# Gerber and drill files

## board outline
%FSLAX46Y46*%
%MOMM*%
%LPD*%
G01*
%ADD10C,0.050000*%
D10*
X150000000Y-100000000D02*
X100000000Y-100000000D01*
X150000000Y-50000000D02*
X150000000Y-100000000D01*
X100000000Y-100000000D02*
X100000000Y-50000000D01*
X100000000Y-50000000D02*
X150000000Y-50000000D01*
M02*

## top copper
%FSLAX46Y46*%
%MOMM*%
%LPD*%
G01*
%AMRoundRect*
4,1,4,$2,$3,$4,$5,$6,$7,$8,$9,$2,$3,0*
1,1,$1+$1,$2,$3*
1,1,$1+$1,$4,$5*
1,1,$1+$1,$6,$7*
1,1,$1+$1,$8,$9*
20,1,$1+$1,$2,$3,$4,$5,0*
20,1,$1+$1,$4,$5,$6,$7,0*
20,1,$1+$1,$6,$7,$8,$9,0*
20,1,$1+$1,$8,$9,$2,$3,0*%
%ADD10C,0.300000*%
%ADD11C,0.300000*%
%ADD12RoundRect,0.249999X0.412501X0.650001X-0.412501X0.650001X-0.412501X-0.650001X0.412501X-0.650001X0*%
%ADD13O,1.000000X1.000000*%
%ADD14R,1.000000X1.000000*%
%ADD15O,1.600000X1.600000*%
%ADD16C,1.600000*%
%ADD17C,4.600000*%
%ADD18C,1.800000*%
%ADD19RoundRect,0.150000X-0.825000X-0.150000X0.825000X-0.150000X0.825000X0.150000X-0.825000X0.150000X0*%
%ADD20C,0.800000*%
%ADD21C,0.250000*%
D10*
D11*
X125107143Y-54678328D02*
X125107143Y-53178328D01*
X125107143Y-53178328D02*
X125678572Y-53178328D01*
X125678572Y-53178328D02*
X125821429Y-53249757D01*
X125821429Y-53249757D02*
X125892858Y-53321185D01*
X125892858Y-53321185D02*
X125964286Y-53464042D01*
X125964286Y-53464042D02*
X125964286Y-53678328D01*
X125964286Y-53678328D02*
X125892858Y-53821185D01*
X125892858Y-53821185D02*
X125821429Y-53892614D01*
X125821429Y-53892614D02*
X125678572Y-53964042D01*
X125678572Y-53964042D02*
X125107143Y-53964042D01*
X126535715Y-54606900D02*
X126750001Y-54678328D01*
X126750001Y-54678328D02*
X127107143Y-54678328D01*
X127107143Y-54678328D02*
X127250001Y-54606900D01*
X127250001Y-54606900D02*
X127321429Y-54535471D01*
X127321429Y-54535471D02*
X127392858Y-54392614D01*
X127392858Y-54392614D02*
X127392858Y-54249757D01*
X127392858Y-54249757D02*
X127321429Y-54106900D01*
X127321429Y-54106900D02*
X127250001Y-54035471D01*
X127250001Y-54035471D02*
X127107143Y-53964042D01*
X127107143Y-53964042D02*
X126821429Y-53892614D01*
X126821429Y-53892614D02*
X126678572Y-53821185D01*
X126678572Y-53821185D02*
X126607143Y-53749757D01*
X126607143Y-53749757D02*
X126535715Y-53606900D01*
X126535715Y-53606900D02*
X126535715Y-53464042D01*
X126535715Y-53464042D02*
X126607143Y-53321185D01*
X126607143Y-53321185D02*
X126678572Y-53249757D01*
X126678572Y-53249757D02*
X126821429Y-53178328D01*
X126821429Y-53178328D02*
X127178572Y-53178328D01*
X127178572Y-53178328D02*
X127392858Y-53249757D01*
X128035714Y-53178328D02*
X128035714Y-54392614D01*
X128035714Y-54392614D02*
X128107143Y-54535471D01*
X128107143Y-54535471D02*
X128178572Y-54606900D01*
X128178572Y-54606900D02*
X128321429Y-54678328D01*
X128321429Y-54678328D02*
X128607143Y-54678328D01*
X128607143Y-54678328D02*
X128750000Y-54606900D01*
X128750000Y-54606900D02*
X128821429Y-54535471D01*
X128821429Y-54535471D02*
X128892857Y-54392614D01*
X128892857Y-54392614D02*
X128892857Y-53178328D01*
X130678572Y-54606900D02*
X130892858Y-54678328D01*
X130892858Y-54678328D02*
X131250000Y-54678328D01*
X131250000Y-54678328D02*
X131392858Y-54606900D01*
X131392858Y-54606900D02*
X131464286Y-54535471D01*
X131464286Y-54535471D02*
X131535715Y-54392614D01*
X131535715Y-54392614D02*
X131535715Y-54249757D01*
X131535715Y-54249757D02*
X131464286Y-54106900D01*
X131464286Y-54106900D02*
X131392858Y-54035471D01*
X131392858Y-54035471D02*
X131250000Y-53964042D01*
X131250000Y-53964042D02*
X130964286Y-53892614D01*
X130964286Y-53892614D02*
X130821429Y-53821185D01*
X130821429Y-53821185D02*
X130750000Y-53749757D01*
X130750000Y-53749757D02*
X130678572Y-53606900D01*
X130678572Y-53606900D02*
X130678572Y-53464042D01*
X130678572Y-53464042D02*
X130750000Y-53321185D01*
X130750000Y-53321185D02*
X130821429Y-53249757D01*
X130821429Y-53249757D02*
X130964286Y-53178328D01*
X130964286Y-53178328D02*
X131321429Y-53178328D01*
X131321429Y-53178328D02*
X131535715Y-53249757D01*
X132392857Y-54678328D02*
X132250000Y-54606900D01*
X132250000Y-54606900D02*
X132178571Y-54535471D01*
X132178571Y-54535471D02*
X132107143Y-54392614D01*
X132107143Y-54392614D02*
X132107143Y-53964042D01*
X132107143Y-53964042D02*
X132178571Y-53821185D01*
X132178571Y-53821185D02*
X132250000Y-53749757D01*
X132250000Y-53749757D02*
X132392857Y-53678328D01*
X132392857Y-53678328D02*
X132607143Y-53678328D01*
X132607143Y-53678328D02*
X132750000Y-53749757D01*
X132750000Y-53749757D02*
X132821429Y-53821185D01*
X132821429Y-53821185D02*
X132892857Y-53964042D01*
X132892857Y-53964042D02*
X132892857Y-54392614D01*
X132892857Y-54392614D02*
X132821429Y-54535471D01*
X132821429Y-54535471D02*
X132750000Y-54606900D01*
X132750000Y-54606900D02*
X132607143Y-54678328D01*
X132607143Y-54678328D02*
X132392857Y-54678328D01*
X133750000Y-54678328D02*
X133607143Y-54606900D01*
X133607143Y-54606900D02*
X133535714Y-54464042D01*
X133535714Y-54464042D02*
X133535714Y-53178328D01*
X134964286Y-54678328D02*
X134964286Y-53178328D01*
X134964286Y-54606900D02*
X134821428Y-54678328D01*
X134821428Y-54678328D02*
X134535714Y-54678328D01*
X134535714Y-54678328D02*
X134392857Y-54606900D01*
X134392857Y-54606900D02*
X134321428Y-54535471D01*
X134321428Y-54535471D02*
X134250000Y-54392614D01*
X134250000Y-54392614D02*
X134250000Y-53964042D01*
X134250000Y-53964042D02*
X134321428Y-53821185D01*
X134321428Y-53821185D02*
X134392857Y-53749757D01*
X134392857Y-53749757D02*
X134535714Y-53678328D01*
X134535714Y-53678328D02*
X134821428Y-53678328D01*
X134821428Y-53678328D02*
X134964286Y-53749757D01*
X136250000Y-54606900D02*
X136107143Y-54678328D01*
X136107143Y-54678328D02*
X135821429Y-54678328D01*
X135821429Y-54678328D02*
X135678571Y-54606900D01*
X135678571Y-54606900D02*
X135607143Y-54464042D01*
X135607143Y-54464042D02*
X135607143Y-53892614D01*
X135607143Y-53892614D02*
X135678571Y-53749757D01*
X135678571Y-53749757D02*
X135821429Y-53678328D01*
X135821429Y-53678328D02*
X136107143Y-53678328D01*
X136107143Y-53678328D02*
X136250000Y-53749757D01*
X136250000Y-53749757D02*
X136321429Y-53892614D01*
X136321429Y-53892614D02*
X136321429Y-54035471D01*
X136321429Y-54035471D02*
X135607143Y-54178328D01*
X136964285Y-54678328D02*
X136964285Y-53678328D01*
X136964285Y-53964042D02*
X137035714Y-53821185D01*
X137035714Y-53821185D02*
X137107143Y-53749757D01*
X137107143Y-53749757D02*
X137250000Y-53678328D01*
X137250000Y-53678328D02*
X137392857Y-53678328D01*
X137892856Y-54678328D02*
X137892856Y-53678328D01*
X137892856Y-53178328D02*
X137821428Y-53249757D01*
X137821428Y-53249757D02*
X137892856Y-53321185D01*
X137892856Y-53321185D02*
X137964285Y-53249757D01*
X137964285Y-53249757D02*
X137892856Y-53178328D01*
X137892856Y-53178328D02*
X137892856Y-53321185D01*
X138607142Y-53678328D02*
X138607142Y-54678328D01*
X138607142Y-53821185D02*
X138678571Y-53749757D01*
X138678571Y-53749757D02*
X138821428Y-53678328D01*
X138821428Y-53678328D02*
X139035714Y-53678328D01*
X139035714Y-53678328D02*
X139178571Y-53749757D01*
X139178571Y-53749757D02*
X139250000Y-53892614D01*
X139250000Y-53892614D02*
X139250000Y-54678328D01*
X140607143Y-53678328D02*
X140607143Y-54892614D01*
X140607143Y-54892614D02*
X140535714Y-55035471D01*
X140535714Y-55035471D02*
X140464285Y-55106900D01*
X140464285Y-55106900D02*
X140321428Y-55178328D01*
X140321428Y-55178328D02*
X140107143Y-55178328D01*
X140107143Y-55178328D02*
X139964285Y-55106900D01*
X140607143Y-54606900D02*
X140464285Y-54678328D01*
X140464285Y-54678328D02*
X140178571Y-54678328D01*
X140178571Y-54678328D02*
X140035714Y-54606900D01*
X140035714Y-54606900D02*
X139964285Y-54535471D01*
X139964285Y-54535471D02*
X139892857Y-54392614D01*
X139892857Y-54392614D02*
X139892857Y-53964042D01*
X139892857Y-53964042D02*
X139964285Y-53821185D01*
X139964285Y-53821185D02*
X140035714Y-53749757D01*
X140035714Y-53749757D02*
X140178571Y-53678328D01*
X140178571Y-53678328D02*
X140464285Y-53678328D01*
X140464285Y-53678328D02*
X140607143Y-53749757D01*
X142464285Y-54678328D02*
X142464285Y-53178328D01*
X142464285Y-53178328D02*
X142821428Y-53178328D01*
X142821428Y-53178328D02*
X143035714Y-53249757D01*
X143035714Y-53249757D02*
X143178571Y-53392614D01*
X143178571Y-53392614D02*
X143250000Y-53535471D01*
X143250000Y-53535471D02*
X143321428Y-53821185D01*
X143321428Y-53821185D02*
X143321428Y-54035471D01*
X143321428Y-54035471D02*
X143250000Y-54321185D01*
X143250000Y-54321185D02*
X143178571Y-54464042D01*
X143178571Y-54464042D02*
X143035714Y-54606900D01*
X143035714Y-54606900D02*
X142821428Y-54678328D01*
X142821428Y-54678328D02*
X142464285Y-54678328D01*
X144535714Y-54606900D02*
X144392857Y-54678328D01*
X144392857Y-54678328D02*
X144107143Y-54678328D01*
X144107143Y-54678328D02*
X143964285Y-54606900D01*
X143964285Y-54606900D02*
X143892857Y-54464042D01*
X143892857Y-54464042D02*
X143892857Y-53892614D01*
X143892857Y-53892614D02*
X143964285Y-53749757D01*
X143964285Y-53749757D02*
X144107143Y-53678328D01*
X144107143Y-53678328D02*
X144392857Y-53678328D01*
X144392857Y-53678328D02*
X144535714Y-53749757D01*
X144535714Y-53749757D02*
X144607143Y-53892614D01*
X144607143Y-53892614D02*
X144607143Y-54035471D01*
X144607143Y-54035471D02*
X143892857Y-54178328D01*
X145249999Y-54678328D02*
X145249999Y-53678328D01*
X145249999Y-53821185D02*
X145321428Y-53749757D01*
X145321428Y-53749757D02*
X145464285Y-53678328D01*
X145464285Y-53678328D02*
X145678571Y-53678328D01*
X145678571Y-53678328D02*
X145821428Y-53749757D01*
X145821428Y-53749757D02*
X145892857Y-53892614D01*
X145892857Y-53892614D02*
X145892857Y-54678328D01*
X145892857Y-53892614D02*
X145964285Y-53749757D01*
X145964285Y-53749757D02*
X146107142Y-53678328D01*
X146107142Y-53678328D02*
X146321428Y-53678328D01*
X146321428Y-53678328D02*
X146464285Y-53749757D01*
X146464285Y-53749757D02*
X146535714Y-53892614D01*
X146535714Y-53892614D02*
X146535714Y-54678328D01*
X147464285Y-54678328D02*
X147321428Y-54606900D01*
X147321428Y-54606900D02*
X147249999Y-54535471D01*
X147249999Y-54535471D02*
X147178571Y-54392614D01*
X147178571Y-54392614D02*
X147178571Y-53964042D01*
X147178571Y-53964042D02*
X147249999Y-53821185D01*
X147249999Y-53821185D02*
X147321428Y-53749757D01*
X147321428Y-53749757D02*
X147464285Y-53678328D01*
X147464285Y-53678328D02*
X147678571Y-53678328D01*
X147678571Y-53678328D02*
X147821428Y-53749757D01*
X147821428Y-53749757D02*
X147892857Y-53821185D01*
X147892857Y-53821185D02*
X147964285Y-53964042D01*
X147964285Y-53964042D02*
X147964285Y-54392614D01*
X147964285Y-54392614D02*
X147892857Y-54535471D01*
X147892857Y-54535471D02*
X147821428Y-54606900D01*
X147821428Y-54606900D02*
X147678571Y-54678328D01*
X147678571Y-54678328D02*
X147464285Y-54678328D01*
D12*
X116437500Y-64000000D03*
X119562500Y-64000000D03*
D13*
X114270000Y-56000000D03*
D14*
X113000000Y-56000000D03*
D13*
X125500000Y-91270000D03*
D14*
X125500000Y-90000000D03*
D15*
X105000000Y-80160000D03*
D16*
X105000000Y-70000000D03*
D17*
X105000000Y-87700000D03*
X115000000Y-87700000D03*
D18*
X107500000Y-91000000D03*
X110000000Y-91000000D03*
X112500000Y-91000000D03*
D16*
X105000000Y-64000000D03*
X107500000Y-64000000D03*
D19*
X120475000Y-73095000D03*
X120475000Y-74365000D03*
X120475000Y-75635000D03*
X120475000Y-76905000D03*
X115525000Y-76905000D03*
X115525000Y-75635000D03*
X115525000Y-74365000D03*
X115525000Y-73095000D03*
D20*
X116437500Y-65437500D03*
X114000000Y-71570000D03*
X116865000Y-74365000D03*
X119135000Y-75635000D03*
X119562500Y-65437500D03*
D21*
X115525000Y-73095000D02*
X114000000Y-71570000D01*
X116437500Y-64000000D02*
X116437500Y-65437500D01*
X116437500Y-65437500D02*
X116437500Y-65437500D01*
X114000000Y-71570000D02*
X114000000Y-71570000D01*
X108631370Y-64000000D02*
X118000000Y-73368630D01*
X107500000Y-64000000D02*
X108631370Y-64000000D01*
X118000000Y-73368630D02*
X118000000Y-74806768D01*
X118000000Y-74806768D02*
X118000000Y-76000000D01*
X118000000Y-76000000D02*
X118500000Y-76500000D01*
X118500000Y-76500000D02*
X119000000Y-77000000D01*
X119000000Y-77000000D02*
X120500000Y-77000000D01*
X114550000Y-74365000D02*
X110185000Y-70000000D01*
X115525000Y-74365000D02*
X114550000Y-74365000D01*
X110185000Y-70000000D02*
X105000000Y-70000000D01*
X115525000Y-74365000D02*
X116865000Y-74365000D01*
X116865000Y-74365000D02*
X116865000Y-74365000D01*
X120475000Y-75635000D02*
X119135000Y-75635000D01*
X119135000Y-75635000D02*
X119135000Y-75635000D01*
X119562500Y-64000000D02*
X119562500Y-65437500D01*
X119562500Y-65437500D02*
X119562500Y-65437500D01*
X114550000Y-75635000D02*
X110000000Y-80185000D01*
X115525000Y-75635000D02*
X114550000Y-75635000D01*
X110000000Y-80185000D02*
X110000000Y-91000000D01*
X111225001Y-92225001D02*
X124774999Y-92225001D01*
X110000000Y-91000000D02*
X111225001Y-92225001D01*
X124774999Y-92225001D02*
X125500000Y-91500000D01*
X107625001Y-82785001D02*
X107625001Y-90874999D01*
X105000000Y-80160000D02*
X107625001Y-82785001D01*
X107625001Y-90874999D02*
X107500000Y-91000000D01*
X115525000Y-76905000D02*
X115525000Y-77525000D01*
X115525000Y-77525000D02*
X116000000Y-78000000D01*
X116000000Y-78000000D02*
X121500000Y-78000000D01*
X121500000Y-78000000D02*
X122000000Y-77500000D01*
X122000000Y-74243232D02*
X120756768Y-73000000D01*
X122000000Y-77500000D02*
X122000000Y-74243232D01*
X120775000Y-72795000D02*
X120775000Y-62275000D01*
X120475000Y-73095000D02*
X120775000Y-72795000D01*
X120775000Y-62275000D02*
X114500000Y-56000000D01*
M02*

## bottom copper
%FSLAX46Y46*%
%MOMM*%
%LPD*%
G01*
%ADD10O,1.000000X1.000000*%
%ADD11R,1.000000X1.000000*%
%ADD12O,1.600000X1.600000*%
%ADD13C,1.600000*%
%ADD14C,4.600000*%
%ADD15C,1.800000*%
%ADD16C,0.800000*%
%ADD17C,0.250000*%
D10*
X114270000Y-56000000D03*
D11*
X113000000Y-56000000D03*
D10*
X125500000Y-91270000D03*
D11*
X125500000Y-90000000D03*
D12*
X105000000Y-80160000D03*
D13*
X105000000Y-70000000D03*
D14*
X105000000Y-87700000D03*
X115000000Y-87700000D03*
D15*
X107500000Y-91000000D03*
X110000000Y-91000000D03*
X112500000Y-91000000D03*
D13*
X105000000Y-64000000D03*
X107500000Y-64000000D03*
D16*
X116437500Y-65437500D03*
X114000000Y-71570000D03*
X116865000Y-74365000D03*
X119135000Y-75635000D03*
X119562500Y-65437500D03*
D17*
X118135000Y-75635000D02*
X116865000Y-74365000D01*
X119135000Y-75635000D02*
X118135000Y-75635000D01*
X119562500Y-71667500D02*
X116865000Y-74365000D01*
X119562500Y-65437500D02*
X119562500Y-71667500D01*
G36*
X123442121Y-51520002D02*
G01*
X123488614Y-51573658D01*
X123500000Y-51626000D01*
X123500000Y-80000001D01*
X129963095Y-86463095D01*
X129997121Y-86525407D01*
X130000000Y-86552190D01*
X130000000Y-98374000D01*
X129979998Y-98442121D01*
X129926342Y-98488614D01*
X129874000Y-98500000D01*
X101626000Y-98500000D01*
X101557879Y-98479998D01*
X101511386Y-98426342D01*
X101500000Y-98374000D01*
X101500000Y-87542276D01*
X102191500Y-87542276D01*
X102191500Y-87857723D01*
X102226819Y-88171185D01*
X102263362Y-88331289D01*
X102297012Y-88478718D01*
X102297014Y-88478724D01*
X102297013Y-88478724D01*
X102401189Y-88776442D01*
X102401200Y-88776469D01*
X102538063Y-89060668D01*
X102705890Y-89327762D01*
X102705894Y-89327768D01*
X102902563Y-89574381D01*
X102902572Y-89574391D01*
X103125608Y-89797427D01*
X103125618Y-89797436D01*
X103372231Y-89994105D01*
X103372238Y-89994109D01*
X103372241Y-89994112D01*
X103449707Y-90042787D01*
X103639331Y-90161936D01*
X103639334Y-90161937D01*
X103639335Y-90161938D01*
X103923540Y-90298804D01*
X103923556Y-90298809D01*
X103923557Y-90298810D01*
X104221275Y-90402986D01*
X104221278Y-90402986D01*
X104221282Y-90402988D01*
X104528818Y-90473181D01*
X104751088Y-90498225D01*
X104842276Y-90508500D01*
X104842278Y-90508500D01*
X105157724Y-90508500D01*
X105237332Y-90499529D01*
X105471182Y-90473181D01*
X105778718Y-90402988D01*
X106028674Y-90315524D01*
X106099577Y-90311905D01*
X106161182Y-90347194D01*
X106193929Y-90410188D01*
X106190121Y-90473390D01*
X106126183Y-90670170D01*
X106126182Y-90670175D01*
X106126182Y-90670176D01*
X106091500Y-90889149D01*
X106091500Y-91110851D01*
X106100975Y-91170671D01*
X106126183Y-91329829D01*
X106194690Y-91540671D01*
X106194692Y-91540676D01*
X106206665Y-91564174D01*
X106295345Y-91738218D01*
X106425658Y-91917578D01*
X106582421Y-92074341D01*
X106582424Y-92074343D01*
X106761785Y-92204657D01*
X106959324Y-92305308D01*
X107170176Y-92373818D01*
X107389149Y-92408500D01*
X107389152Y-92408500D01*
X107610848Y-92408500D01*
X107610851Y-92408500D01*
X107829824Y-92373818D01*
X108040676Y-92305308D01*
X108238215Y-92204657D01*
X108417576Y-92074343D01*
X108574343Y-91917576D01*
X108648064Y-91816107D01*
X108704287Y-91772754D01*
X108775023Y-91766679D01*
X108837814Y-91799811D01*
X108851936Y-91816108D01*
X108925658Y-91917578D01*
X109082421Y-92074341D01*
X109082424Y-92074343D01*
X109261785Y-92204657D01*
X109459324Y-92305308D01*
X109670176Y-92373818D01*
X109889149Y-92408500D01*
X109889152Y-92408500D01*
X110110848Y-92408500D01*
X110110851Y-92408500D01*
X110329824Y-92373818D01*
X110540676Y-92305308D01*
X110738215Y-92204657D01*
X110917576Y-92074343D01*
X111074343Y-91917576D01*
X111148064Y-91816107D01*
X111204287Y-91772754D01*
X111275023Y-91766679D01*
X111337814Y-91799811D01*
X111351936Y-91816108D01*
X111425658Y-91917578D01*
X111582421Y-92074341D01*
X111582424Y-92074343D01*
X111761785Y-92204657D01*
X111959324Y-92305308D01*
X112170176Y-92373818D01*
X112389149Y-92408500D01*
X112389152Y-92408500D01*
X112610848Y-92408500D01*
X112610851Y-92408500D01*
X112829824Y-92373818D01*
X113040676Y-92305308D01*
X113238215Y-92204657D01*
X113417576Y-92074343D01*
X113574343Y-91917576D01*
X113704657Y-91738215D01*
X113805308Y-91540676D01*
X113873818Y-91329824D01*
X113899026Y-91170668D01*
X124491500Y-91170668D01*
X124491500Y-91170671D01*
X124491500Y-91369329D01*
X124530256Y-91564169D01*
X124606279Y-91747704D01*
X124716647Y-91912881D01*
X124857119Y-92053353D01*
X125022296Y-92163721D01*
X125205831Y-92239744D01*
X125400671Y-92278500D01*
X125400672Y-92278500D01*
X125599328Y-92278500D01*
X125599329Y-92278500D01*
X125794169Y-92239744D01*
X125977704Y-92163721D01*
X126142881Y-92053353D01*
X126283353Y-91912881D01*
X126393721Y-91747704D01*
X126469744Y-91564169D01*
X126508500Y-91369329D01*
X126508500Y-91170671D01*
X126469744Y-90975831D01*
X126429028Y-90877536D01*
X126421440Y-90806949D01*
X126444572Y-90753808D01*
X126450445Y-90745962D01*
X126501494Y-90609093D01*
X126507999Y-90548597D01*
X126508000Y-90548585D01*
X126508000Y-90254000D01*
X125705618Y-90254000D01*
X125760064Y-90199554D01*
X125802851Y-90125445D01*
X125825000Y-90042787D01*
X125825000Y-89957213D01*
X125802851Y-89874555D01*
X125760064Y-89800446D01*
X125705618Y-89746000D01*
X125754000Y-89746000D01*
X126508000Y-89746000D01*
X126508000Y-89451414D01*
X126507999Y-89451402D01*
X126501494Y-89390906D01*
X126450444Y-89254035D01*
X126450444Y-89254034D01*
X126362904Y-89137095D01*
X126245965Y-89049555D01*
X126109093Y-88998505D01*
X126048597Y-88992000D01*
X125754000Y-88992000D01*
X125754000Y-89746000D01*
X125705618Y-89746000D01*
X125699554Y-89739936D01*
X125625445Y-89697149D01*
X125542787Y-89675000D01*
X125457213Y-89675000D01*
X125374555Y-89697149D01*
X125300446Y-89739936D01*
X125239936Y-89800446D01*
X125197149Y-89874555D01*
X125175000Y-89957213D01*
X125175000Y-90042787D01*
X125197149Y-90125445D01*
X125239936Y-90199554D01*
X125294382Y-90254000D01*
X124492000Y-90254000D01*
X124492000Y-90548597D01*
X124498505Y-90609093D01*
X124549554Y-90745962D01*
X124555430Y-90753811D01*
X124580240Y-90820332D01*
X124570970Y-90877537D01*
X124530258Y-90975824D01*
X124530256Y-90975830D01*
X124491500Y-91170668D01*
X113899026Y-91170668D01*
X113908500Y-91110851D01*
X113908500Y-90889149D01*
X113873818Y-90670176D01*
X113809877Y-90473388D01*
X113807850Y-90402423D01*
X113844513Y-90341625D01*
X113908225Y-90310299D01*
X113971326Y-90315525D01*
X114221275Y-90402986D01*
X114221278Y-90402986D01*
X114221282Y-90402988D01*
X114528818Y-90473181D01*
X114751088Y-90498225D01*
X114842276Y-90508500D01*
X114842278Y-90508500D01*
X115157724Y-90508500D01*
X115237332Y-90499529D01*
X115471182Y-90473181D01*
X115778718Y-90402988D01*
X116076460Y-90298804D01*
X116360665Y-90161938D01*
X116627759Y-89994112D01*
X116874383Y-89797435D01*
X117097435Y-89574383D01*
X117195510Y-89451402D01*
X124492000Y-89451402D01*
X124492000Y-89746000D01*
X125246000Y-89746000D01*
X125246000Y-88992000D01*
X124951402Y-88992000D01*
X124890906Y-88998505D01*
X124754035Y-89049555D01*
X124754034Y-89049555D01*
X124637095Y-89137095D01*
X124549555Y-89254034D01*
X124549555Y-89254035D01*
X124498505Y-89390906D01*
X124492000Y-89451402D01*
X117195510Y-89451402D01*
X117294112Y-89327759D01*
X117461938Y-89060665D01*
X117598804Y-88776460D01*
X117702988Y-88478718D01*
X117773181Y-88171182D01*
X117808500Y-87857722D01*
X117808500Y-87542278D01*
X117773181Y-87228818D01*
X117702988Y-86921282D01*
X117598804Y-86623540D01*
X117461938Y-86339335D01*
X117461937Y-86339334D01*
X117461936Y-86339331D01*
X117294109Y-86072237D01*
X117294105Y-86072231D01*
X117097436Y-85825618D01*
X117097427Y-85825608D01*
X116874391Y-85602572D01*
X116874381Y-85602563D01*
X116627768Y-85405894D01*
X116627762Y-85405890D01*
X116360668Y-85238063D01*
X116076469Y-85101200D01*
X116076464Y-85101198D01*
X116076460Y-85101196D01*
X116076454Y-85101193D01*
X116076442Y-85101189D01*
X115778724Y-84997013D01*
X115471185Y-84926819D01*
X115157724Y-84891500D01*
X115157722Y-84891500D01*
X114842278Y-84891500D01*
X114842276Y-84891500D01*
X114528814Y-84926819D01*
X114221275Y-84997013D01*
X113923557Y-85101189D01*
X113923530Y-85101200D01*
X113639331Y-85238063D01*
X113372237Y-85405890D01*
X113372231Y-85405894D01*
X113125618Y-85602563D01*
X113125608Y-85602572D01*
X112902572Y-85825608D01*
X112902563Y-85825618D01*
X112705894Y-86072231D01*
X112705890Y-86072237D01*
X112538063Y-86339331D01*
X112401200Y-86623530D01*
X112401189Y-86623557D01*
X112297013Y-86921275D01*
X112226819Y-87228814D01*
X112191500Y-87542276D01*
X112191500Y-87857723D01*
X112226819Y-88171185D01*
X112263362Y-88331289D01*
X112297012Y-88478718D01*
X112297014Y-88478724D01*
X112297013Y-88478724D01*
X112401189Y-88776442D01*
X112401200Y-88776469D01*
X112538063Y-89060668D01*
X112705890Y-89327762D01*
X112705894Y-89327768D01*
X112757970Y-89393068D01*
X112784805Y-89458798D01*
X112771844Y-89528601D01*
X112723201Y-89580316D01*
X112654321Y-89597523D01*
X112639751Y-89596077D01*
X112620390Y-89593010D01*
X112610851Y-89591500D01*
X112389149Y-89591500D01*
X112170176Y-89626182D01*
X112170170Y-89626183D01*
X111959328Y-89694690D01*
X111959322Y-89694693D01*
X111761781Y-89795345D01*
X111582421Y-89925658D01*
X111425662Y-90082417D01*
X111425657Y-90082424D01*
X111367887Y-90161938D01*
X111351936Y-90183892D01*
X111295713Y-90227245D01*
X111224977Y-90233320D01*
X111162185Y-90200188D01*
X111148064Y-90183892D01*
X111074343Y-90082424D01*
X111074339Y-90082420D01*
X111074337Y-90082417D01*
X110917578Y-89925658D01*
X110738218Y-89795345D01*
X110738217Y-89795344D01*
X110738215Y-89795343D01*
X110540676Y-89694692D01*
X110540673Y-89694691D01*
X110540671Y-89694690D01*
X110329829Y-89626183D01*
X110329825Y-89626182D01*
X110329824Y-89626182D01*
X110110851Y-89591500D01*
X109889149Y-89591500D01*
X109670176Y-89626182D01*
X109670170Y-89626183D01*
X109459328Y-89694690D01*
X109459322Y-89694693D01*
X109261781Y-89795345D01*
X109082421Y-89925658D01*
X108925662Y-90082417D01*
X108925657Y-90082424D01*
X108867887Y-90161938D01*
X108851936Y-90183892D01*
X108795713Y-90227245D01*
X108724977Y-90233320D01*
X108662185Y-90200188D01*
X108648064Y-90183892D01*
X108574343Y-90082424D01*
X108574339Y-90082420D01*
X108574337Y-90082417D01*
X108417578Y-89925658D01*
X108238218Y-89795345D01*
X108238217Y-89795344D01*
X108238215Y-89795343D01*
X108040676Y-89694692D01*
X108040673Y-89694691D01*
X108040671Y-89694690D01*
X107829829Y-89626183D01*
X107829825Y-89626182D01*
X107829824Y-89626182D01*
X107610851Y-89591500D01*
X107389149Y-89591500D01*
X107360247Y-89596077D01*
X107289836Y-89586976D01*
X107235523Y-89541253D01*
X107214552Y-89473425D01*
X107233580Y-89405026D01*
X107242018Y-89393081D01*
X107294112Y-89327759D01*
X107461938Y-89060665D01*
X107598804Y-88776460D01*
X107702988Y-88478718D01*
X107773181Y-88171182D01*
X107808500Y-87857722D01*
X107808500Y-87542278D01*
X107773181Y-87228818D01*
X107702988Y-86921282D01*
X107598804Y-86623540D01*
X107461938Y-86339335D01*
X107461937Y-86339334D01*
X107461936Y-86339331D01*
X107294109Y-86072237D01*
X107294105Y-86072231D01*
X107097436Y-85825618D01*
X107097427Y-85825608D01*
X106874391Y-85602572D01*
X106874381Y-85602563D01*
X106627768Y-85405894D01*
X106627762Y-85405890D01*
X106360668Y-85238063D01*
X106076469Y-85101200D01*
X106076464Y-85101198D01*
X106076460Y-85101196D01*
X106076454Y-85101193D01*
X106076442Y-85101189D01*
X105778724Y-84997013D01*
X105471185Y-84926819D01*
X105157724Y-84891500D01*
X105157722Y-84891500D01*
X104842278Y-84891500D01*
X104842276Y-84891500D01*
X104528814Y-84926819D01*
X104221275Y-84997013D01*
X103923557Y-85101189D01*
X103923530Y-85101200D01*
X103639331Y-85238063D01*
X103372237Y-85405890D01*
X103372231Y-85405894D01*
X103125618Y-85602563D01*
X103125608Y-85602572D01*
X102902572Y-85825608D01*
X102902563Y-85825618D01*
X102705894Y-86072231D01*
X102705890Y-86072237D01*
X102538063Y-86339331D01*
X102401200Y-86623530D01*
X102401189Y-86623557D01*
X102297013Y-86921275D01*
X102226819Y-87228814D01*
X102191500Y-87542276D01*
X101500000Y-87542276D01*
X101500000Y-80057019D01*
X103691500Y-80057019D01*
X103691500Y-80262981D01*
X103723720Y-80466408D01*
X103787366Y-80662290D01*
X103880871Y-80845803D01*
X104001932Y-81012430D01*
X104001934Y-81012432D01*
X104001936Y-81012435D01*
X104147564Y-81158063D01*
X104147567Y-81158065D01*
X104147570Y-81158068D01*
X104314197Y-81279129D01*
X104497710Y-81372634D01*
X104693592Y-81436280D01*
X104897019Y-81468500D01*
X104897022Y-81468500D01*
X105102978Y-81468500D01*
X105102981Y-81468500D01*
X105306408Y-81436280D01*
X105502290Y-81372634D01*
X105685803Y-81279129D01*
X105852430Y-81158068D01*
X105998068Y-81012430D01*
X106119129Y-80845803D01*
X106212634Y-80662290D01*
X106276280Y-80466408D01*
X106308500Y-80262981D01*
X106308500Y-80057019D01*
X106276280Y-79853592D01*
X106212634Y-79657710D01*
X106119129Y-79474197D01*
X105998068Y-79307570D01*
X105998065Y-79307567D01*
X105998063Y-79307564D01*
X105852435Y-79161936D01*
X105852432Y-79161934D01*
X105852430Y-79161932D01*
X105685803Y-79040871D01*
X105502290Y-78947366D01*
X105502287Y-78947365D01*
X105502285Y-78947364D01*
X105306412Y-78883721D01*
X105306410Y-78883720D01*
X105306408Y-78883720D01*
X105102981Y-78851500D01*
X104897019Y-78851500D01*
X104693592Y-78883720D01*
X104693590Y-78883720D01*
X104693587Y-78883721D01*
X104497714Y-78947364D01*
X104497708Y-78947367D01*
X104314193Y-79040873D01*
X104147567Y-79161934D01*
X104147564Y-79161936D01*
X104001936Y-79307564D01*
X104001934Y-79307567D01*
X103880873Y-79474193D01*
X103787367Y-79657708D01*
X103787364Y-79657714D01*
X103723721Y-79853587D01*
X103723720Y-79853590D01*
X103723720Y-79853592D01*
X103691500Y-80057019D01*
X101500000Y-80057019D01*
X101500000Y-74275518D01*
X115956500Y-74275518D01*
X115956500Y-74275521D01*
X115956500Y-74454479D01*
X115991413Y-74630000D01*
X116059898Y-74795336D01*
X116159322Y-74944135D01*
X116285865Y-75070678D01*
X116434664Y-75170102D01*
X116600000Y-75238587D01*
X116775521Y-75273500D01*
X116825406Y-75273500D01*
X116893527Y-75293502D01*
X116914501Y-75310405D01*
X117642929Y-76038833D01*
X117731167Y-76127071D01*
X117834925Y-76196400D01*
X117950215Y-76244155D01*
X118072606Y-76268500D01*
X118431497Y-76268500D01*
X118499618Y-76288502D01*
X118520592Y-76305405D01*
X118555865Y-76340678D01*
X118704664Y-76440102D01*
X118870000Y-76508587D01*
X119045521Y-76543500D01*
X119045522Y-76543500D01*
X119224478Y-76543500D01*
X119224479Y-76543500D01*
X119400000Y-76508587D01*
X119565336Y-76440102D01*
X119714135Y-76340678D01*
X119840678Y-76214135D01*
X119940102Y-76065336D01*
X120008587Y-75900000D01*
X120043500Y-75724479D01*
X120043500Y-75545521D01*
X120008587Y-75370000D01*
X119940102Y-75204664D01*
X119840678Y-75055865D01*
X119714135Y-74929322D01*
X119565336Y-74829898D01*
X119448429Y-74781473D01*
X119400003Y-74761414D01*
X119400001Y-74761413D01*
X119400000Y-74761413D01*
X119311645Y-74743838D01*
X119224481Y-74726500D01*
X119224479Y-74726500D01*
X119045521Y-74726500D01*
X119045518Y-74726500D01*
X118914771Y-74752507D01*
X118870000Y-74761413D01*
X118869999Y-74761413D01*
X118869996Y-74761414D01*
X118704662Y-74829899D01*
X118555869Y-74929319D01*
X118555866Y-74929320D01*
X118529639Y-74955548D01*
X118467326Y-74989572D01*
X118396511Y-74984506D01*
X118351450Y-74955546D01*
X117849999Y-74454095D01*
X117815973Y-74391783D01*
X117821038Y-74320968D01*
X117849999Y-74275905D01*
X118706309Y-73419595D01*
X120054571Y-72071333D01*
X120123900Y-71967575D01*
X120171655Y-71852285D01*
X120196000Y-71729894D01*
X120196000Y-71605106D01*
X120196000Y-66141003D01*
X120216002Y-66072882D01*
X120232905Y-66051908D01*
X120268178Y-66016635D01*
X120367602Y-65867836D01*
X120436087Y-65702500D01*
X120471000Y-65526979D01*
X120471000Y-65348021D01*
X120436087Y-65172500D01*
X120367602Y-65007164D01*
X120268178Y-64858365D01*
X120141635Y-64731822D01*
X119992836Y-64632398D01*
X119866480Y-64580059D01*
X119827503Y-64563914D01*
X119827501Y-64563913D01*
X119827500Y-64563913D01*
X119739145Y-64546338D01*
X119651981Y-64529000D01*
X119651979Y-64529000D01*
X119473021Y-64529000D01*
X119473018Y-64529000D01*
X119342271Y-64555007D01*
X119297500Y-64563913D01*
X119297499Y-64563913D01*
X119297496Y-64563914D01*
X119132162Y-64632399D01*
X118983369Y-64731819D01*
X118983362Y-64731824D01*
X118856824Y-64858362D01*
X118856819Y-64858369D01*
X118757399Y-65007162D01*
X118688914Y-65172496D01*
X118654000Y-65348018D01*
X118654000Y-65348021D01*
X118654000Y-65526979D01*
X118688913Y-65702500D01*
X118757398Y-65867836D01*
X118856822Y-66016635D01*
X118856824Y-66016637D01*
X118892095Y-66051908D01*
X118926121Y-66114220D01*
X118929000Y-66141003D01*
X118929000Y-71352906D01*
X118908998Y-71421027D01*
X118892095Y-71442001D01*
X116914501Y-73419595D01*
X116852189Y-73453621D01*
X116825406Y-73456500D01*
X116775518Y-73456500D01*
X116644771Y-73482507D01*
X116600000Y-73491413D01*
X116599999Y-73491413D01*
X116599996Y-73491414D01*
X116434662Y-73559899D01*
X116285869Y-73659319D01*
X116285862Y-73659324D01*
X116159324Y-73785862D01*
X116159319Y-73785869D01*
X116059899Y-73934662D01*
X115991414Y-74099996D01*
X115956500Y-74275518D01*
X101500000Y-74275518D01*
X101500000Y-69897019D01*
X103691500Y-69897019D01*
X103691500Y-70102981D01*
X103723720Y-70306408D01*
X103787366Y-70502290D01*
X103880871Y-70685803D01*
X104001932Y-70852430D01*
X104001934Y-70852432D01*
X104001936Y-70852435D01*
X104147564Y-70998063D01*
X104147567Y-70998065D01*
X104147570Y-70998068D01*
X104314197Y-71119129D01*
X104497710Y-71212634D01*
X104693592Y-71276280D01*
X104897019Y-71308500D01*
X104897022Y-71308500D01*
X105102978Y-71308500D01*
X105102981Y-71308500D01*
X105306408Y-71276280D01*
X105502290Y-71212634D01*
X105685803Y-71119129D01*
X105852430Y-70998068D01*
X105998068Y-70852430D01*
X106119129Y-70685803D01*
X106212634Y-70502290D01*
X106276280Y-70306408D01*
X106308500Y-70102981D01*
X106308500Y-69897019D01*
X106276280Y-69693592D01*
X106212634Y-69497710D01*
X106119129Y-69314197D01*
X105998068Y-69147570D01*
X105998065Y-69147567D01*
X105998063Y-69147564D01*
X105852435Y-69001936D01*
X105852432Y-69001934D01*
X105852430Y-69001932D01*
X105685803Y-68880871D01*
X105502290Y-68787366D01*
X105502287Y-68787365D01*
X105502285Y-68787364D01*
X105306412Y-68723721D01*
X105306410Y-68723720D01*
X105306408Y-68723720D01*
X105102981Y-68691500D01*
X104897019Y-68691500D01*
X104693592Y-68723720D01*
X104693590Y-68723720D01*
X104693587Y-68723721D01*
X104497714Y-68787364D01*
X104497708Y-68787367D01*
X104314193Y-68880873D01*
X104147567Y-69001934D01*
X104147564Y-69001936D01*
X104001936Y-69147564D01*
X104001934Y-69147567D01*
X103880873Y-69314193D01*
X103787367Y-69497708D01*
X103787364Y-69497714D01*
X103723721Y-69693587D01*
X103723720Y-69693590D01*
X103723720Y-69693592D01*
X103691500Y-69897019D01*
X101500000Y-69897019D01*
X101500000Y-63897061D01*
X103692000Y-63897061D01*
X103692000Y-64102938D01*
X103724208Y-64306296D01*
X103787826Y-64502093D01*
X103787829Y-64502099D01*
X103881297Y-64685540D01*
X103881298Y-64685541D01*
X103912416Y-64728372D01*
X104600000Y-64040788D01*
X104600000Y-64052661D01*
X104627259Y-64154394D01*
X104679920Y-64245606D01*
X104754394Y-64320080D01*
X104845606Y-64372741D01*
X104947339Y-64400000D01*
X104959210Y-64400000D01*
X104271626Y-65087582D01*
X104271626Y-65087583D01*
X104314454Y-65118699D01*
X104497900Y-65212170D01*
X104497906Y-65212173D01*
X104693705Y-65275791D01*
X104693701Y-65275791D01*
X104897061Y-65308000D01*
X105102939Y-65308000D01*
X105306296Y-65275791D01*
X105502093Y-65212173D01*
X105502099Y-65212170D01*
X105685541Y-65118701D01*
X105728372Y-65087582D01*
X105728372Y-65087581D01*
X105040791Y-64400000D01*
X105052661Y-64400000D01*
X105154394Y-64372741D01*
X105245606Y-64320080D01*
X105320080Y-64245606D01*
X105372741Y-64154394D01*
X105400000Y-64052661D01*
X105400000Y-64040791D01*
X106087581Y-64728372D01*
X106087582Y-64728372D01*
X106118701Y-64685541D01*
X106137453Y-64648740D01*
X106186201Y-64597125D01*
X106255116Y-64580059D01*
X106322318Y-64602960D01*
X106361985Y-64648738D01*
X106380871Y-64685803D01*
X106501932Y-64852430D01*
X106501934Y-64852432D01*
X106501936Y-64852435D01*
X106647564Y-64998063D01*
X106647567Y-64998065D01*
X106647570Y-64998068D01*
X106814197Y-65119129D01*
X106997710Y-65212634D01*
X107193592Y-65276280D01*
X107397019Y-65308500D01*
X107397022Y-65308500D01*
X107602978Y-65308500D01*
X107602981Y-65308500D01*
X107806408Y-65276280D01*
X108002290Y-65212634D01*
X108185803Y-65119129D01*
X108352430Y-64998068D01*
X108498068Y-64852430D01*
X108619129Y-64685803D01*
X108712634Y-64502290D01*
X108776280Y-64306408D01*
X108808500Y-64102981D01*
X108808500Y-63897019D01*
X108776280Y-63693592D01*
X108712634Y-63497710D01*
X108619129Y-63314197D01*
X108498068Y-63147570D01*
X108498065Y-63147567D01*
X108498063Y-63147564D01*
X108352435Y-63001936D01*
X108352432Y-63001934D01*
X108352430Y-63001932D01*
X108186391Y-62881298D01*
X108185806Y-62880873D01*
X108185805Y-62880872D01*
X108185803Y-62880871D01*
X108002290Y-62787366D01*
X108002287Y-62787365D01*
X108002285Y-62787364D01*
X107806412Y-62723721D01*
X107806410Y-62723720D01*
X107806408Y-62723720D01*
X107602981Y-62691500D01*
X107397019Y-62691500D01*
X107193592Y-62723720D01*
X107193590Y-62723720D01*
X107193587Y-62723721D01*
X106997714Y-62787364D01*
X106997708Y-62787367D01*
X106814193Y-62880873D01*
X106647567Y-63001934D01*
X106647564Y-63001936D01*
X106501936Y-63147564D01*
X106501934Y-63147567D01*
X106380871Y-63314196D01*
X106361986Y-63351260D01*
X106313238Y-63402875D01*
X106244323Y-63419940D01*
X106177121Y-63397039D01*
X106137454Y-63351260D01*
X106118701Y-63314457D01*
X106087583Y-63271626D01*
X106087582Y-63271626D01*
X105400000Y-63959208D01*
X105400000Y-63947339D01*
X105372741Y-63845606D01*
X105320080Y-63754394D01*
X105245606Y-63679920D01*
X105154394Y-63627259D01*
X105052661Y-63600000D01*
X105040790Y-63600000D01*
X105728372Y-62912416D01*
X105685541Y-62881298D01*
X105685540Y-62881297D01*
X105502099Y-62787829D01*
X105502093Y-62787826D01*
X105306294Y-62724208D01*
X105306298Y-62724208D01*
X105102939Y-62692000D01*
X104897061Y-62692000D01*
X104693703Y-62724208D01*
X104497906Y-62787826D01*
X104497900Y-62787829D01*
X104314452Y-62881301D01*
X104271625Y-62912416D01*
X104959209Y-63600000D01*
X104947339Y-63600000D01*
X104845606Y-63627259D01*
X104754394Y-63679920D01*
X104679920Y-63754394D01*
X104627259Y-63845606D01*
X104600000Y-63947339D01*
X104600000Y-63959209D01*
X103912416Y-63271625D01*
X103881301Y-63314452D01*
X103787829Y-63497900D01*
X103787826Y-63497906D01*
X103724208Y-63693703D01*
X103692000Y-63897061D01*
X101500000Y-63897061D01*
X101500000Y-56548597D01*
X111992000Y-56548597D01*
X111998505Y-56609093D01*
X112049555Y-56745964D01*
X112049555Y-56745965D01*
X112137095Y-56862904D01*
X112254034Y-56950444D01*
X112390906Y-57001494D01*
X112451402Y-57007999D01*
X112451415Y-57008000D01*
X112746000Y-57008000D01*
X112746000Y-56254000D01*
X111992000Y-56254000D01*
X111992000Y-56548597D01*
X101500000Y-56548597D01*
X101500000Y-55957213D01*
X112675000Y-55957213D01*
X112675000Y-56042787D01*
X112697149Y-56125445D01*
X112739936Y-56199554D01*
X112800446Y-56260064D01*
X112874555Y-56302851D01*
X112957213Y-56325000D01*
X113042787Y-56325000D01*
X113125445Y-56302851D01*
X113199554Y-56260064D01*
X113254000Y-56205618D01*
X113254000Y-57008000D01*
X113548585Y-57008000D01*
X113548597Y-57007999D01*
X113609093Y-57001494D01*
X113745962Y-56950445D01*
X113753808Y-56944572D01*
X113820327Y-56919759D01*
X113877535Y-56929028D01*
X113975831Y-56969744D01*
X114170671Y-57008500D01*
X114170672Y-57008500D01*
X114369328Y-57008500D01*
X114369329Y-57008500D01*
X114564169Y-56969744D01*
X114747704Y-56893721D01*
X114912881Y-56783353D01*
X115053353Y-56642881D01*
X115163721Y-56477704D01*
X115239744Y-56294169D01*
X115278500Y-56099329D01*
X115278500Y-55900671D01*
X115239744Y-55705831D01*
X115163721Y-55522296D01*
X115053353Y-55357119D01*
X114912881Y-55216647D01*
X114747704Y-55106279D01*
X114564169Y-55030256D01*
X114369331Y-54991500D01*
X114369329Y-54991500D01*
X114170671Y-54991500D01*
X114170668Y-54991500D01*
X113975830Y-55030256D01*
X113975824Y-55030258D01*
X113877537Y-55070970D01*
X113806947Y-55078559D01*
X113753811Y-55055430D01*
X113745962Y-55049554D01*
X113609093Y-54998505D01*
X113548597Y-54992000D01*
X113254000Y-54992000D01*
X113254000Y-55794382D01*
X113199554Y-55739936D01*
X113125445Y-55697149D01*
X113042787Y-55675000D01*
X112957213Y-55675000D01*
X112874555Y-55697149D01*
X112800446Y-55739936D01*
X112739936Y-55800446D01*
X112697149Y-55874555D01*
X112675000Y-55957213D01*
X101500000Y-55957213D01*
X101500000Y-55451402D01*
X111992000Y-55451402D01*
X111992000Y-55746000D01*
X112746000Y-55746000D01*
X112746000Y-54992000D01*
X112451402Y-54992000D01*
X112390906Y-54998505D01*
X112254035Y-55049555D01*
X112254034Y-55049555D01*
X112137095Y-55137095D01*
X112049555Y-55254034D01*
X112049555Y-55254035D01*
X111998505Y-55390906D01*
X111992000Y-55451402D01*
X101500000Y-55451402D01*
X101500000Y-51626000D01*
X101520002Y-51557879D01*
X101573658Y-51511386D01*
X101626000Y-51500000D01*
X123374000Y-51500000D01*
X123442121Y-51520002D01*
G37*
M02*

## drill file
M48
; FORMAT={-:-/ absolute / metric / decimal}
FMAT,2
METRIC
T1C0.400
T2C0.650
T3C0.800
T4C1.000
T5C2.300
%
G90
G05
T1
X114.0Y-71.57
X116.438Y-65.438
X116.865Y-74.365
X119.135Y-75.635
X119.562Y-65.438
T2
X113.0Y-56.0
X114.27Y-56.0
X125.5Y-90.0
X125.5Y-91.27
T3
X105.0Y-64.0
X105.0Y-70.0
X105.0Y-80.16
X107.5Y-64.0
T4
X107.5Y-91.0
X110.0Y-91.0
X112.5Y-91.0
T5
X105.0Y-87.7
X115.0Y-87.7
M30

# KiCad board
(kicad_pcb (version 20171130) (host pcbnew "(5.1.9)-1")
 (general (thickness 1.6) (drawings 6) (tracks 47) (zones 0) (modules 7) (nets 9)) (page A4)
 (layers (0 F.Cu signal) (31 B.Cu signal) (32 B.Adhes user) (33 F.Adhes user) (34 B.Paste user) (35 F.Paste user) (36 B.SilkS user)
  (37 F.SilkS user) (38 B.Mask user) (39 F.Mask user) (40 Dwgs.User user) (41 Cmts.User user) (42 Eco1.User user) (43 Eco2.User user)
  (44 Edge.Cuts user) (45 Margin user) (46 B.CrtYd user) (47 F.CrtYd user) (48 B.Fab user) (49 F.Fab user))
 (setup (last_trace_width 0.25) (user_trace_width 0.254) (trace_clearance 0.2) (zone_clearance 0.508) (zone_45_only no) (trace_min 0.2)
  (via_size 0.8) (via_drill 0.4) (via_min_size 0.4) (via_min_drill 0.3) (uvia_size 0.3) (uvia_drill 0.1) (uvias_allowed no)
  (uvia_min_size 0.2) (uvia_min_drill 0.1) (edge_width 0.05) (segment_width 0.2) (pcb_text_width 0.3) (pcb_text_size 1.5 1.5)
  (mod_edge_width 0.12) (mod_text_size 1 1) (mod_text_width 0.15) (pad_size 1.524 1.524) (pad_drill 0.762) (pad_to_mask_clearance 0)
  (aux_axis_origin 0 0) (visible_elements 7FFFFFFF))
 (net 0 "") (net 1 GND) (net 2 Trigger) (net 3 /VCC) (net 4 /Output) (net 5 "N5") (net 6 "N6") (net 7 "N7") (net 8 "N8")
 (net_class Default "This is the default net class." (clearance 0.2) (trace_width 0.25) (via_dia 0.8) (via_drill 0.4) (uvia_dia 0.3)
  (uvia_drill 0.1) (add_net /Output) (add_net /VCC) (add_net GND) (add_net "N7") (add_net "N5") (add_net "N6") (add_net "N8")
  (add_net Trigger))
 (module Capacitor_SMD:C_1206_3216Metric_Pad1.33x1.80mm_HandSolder (layer F.Cu) (at 118 64 180)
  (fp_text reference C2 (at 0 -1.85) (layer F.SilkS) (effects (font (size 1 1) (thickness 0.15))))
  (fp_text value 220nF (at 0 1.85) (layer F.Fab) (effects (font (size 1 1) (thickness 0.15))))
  (pad 2 smd roundrect (at 1.5625 0 180) (size 1.325 1.8) (layers F.Cu F.Paste F.Mask) (roundrect_rratio 0.1886784905660377) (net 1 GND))
  (pad 1 smd roundrect (at -1.5625 0 180) (size 1.325 1.8) (layers F.Cu F.Paste F.Mask) (roundrect_rratio 0.1886784905660377)
   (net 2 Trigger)))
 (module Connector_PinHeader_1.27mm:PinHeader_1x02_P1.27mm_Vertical (layer F.Cu) (at 113 56 90)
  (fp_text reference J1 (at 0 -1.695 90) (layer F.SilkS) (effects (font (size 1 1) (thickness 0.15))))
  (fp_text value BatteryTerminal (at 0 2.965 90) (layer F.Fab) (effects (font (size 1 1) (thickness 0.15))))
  (pad 2 thru_hole oval (at 0 1.27 90) (size 1 1) (drill 0.65) (layers *.Cu *.Mask) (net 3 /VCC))
  (pad 1 thru_hole rect (at 0 0 90) (size 1 1) (drill 0.65) (layers *.Cu *.Mask) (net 1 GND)))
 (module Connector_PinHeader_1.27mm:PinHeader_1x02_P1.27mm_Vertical (layer F.Cu) (at 125.5 90)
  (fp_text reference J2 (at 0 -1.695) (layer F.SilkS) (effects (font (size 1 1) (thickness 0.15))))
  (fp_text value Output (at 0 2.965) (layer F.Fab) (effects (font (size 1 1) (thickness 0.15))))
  (pad 2 thru_hole oval (at 0 1.27) (size 1 1) (drill 0.65) (layers *.Cu *.Mask) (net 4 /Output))
  (pad 1 thru_hole rect (at 0 0) (size 1 1) (drill 0.65) (layers *.Cu *.Mask) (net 1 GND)))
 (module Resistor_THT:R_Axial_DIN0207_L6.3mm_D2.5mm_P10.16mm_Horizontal (layer F.Cu) (at 105 70 270)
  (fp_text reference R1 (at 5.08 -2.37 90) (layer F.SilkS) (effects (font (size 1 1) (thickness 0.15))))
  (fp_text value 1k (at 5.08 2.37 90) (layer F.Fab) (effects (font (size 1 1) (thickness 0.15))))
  (pad 2 thru_hole oval (at 10.16 0 270) (size 1.6 1.6) (drill 0.8) (layers *.Cu *.Mask) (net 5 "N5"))
  (pad 1 thru_hole circle (at 0 0 270) (size 1.6 1.6) (drill 0.8) (layers *.Cu *.Mask) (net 2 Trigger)))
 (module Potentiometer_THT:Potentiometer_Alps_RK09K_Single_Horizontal (layer F.Cu) (at 107.5 91 270)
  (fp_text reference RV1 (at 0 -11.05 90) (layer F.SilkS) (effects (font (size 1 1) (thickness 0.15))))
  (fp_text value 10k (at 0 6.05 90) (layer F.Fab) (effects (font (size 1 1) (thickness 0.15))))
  (pad "" thru_hole circle (at -3.3 2.5 270) (size 4.6 4.6) (drill 2.3) (layers *.Cu *.Mask))
  (pad "" thru_hole circle (at -3.3 -7.5 270) (size 4.6 4.6) (drill 2.3) (layers *.Cu *.Mask))
  (pad 1 thru_hole circle (at 0 0 270) (size 1.8 1.8) (drill 1) (layers *.Cu *.Mask) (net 5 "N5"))
  (pad 2 thru_hole circle (at 0 -2.5 270) (size 1.8 1.8) (drill 1) (layers *.Cu *.Mask) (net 4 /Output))
  (pad 3 thru_hole circle (at 0 -5 270) (size 1.8 1.8) (drill 1) (layers *.Cu *.Mask) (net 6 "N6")))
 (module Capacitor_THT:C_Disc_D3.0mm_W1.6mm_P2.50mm (layer F.Cu) (at 107.5 64 180)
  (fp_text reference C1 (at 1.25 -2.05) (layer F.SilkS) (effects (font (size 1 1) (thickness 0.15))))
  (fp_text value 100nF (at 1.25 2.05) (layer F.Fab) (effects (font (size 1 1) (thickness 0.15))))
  (pad 2 thru_hole circle (at 2.5 0 180) (size 1.6 1.6) (drill 0.8) (layers *.Cu *.Mask) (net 1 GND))
  (pad 1 thru_hole circle (at 0 0 180) (size 1.6 1.6) (drill 0.8) (layers *.Cu *.Mask) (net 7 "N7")))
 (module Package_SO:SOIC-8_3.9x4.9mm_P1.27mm (layer F.Cu) (at 118 75)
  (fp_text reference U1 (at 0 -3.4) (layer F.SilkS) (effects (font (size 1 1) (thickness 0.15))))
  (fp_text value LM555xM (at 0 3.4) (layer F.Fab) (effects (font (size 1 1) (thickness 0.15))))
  (pad 8 smd roundrect (at 2.475 -1.905) (size 1.95 0.6) (layers F.Cu F.Paste F.Mask) (roundrect_rratio 0.25) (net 3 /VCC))
  (pad 7 smd roundrect (at 2.475 -0.635) (size 1.95 0.6) (layers F.Cu F.Paste F.Mask) (roundrect_rratio 0.25) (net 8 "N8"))
  (pad 6 smd roundrect (at 2.475 0.635) (size 1.95 0.6) (layers F.Cu F.Paste F.Mask) (roundrect_rratio 0.25) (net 2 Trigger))
  (pad 5 smd roundrect (at 2.475 1.905) (size 1.95 0.6) (layers F.Cu F.Paste F.Mask) (roundrect_rratio 0.25) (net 7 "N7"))
  (pad 4 smd roundrect (at -2.475 1.905) (size 1.95 0.6) (layers F.Cu F.Paste F.Mask) (roundrect_rratio 0.25) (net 3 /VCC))
  (pad 3 smd roundrect (at -2.475 0.635) (size 1.95 0.6) (layers F.Cu F.Paste F.Mask) (roundrect_rratio 0.25) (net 4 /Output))
  (pad 2 smd roundrect (at -2.475 -0.635) (size 1.95 0.6) (layers F.Cu F.Paste F.Mask) (roundrect_rratio 0.25) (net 2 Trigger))
  (pad 1 smd roundrect (at -2.475 -1.905) (size 1.95 0.6) (layers F.Cu F.Paste F.Mask) (roundrect_rratio 0.25) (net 1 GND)))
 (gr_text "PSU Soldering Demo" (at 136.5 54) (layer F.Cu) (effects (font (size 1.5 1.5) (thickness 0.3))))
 (gr_line (start 150 100) (end 100 100) (layer Edge.Cuts) (width 0.05))
 (gr_line (start 150 50) (end 150 100) (layer Edge.Cuts) (width 0.05))
 (gr_line (start 100 100) (end 100 50) (layer Edge.Cuts) (width 0.05))
 (gr_line (start 100 50) (end 150 50) (layer Edge.Cuts) (width 0.05))
 (segment (start 115.525 73.095) (end 114 71.57) (width 0.25) (layer F.Cu) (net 1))
 (segment (start 116.4375 64) (end 116.4375 65.4375) (width 0.25) (layer F.Cu) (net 1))
 (segment (start 116.4375 65.4375) (end 116.4375 65.4375) (width 0.25) (layer F.Cu) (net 1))
 (via (at 116.4375 65.4375) (size 0.8) (drill 0.4) (layers F.Cu B.Cu) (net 1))
 (segment (start 114 71.57) (end 114 71.57) (width 0.25) (layer F.Cu) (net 1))
 (via (at 114 71.57) (size 0.8) (drill 0.4) (layers F.Cu B.Cu) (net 1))
 (segment (start 108.63137 64) (end 118 73.36863) (width 0.25) (layer F.Cu) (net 7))
 (segment (start 107.5 64) (end 108.63137 64) (width 0.25) (layer F.Cu) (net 7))
 (segment (start 118 73.36863) (end 118 74.806768) (width 0.25) (layer F.Cu) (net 7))
 (segment (start 118 74.806768) (end 118 76) (width 0.25) (layer F.Cu) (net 7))
 (segment (start 118 76) (end 118.5 76.5) (width 0.25) (layer F.Cu) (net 7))
 (segment (start 118.5 76.5) (end 119 77) (width 0.25) (layer F.Cu) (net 7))
 (segment (start 119 77) (end 120.5 77) (width 0.25) (layer F.Cu) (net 7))
 (segment (start 114.55 74.365) (end 110.185 70) (width 0.25) (layer F.Cu) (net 2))
 (segment (start 115.525 74.365) (end 114.55 74.365) (width 0.25) (layer F.Cu) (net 2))
 (segment (start 110.185 70) (end 105 70) (width 0.25) (layer F.Cu) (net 2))
 (segment (start 115.525 74.365) (end 116.865 74.365) (width 0.25) (layer F.Cu) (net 2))
 (segment (start 116.865 74.365) (end 116.865 74.365) (width 0.25) (layer F.Cu) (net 2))
 (via (at 116.865 74.365) (size 0.8) (drill 0.4) (layers F.Cu B.Cu) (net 2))
 (segment (start 120.475 75.635) (end 119.135 75.635) (width 0.25) (layer F.Cu) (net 2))
 (segment (start 119.135 75.635) (end 119.135 75.635) (width 0.25) (layer F.Cu) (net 2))
 (via (at 119.135 75.635) (size 0.8) (drill 0.4) (layers F.Cu B.Cu) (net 2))
 (segment (start 118.135 75.635) (end 116.865 74.365) (width 0.25) (layer B.Cu) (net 2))
 (segment (start 119.135 75.635) (end 118.135 75.635) (width 0.25) (layer B.Cu) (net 2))
 (segment (start 119.5625 64) (end 119.5625 65.4375) (width 0.25) (layer F.Cu) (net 2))
 (segment (start 119.5625 65.4375) (end 119.5625 65.4375) (width 0.25) (layer F.Cu) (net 2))
 (via (at 119.5625 65.4375) (size 0.8) (drill 0.4) (layers F.Cu B.Cu) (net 2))
 (segment (start 119.5625 71.6675) (end 116.865 74.365) (width 0.25) (layer B.Cu) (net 2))
 (segment (start 119.5625 65.4375) (end 119.5625 71.6675) (width 0.25) (layer B.Cu) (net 2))
 (segment (start 114.55 75.635) (end 110 80.185) (width 0.25) (layer F.Cu) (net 4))
 (segment (start 115.525 75.635) (end 114.55 75.635) (width 0.25) (layer F.Cu) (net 4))
 (segment (start 110 80.185) (end 110 91) (width 0.25) (layer F.Cu) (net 4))
 (segment (start 111.225001 92.225001) (end 124.774999 92.225001) (width 0.25) (layer F.Cu) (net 4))
 (segment (start 110 91) (end 111.225001 92.225001) (width 0.25) (layer F.Cu) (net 4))
 (segment (start 124.774999 92.225001) (end 125.5 91.5) (width 0.25) (layer F.Cu) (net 4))
 (segment (start 107.625001 82.785001) (end 107.625001 90.874999) (width 0.25) (layer F.Cu) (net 5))
 (segment (start 105 80.16) (end 107.625001 82.785001) (width 0.25) (layer F.Cu) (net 5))
 (segment (start 107.625001 90.874999) (end 107.5 91) (width 0.25) (layer F.Cu) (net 5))
 (segment (start 115.525 76.905) (end 115.525 77.525) (width 0.25) (layer F.Cu) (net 3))
 (segment (start 115.525 77.525) (end 116 78) (width 0.25) (layer F.Cu) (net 3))
 (segment (start 116 78) (end 121.5 78) (width 0.25) (layer F.Cu) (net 3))
 (segment (start 121.5 78) (end 122 77.5) (width 0.25) (layer F.Cu) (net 3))
 (segment (start 122 74.243232) (end 120.756768 73) (width 0.25) (layer F.Cu) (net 3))
 (segment (start 122 77.5) (end 122 74.243232) (width 0.25) (layer F.Cu) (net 3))
 (segment (start 120.775 72.795) (end 120.775 62.275) (width 0.25) (layer F.Cu) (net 3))
 (segment (start 120.475 73.095) (end 120.775 72.795) (width 0.25) (layer F.Cu) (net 3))
 (segment (start 120.775 62.275) (end 114.5 56) (width 0.25) (layer F.Cu) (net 3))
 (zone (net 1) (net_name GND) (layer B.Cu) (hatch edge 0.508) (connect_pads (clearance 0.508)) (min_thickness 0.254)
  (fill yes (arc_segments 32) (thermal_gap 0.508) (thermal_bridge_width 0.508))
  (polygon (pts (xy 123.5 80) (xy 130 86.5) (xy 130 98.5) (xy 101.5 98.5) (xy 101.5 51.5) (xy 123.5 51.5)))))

